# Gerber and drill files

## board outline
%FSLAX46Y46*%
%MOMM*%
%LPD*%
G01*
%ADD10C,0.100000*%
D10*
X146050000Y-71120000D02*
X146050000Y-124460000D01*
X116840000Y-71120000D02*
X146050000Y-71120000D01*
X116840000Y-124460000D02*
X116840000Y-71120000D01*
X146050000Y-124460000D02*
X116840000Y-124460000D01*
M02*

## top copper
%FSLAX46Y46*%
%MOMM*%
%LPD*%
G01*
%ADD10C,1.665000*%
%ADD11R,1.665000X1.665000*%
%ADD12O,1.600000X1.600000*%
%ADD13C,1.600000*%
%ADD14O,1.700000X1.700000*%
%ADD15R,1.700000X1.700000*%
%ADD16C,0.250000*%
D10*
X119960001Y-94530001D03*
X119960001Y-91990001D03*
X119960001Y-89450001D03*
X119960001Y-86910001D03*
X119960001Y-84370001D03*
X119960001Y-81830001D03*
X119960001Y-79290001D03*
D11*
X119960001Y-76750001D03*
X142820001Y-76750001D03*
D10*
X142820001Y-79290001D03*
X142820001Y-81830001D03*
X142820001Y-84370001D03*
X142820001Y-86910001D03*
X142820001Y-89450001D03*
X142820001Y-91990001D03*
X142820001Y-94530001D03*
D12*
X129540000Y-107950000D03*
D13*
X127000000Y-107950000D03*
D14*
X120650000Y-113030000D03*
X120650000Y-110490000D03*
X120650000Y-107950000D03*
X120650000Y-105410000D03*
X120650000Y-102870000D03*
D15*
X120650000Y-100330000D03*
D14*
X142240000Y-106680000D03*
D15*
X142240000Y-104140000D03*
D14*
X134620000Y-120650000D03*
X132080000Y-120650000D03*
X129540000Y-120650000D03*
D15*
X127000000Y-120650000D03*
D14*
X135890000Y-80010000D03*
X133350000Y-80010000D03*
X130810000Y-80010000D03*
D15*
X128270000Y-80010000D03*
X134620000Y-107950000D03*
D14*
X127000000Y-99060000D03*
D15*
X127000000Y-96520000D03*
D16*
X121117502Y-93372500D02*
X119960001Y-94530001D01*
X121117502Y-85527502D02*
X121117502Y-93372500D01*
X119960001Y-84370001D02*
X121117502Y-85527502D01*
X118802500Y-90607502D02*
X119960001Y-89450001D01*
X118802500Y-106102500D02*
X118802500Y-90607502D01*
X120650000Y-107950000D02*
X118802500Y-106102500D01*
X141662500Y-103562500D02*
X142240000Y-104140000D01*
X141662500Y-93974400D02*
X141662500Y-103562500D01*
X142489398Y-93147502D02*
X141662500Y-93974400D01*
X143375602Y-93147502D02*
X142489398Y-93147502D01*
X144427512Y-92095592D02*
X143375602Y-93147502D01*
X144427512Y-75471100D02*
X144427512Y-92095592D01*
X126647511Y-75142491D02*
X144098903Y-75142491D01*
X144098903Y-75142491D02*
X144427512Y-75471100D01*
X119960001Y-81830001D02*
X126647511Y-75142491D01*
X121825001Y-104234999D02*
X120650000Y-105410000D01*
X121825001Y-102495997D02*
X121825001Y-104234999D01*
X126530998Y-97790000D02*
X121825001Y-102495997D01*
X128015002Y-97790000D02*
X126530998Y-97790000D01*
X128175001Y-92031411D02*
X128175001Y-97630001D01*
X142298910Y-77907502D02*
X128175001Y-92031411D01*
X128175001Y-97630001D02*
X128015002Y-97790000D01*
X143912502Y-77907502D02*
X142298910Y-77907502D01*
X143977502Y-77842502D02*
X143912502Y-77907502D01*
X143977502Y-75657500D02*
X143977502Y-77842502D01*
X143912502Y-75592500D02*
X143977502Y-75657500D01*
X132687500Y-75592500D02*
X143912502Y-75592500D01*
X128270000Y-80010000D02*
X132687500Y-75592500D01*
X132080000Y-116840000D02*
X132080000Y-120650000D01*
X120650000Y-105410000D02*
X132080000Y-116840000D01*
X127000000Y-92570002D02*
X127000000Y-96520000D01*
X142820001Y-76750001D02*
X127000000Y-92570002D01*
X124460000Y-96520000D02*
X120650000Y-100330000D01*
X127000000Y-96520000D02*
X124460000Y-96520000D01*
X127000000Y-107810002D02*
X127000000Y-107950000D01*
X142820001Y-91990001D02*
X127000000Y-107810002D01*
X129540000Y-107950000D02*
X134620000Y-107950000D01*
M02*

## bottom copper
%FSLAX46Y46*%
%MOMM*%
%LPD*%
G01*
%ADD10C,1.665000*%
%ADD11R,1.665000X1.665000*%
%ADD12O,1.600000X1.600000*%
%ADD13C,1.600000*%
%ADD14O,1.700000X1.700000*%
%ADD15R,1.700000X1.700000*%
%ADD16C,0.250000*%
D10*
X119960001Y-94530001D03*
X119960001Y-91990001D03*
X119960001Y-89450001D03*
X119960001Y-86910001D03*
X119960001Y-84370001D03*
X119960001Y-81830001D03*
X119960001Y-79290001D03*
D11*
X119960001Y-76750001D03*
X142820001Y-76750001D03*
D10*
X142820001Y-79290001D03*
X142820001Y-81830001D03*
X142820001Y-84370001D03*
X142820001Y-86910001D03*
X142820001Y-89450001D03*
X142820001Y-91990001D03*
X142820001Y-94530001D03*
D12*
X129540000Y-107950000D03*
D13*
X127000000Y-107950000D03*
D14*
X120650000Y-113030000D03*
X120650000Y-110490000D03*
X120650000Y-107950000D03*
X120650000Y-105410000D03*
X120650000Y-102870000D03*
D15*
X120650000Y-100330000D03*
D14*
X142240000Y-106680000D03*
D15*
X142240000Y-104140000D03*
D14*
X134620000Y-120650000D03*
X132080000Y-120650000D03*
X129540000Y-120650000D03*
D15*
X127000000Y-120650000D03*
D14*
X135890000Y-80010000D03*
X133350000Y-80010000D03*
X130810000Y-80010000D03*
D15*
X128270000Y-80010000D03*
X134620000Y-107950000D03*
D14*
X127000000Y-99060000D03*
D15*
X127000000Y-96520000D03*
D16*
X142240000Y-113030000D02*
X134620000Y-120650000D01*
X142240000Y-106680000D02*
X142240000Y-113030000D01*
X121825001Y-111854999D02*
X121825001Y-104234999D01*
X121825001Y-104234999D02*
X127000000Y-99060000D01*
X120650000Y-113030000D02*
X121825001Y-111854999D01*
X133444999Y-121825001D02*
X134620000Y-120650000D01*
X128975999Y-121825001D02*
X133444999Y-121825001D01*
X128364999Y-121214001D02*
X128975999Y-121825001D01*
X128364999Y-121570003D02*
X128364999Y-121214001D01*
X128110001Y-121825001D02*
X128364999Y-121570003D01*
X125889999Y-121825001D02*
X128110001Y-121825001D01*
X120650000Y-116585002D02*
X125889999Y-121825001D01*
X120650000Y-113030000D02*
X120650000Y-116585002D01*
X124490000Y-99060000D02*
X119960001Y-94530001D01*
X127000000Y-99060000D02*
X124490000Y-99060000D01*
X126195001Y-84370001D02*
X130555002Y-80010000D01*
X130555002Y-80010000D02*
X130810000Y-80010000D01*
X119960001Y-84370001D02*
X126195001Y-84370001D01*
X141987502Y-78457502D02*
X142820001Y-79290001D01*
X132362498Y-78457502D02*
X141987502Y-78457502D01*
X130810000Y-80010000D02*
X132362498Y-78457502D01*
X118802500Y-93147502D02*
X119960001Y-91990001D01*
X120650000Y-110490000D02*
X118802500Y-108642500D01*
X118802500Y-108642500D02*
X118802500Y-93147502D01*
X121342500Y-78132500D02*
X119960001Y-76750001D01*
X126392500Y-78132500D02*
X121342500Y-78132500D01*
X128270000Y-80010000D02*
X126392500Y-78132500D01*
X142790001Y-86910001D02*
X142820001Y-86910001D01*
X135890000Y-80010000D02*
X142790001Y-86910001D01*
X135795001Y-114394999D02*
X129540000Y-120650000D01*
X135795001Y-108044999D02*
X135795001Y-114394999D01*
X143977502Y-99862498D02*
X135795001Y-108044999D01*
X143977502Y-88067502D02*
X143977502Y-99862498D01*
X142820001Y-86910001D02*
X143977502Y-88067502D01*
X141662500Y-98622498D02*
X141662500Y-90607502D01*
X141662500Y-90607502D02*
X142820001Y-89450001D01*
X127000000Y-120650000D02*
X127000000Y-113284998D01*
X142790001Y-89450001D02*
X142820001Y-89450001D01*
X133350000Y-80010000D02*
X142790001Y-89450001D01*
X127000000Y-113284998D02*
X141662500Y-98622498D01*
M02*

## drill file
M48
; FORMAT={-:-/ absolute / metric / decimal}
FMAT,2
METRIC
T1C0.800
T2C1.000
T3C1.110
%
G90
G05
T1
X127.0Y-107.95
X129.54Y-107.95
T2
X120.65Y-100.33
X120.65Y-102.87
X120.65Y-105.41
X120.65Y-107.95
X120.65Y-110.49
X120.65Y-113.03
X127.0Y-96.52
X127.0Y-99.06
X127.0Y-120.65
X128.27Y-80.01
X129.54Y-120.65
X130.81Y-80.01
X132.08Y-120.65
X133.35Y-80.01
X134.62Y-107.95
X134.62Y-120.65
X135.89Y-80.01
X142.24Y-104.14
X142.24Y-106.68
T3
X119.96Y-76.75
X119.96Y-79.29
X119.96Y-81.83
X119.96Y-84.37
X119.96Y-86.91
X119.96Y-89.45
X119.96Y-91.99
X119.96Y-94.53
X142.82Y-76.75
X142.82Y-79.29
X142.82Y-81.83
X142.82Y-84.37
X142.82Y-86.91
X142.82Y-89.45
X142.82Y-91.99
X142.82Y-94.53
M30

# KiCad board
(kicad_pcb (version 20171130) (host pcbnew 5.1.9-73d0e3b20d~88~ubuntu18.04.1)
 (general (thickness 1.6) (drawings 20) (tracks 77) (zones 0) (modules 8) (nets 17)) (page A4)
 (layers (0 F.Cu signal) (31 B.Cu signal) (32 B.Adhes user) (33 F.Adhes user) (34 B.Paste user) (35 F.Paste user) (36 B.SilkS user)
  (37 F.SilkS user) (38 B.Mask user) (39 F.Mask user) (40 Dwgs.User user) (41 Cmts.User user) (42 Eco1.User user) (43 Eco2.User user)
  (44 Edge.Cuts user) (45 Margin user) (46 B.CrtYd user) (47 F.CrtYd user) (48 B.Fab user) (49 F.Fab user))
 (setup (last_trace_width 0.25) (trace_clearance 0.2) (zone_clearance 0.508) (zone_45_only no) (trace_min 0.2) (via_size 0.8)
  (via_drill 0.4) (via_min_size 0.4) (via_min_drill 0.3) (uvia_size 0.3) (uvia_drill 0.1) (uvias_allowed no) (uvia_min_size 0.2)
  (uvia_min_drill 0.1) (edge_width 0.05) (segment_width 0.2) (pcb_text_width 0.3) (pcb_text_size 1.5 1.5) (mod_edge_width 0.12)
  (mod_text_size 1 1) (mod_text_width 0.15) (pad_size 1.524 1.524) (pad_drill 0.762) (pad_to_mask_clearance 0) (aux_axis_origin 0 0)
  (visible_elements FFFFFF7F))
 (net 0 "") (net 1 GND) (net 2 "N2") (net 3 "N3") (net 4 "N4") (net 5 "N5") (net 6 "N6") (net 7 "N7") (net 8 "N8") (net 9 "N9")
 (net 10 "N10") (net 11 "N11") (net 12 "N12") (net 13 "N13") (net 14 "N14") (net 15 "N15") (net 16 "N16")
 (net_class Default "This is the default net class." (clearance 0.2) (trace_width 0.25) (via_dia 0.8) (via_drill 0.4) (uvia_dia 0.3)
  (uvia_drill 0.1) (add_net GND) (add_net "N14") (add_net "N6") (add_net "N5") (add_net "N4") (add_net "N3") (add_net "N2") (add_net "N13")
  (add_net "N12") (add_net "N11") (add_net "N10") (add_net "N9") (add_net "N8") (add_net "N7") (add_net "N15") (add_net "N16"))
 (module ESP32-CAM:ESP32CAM (layer B.Cu) (at 142.820001 94.530001 180)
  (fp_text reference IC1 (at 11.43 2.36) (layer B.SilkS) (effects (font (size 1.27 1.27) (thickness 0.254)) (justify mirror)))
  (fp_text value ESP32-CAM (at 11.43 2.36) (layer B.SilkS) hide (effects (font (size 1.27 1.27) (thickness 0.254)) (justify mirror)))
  (pad 16 thru_hole circle (at 22.86 0 90) (size 1.665 1.665) (drill 1.11) (layers *.Cu *.Mask B.SilkS) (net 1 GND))
  (pad 15 thru_hole circle (at 22.86 2.54 90) (size 1.665 1.665) (drill 1.11) (layers *.Cu *.Mask B.SilkS) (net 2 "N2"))
  (pad 14 thru_hole circle (at 22.86 5.08 90) (size 1.665 1.665) (drill 1.11) (layers *.Cu *.Mask B.SilkS) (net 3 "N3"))
  (pad 13 thru_hole circle (at 22.86 7.62 90) (size 1.665 1.665) (drill 1.11) (layers *.Cu *.Mask B.SilkS) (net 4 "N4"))
  (pad 12 thru_hole circle (at 22.86 10.16 90) (size 1.665 1.665) (drill 1.11) (layers *.Cu *.Mask B.SilkS) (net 1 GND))
  (pad 11 thru_hole circle (at 22.86 12.7 90) (size 1.665 1.665) (drill 1.11) (layers *.Cu *.Mask B.SilkS) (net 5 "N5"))
  (pad 10 thru_hole circle (at 22.86 15.24 90) (size 1.665 1.665) (drill 1.11) (layers *.Cu *.Mask B.SilkS) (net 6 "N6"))
  (pad 9 thru_hole rect (at 22.86 17.78 90) (size 1.665 1.665) (drill 1.11) (layers *.Cu *.Mask B.SilkS) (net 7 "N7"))
  (pad 8 thru_hole rect (at 0 17.78 90) (size 1.665 1.665) (drill 1.11) (layers *.Cu *.Mask B.SilkS) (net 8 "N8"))
  (pad 7 thru_hole circle (at 0 15.24 90) (size 1.665 1.665) (drill 1.11) (layers *.Cu *.Mask B.SilkS) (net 1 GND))
  (pad 6 thru_hole circle (at 0 12.7 90) (size 1.665 1.665) (drill 1.11) (layers *.Cu *.Mask B.SilkS) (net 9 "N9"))
  (pad 5 thru_hole circle (at 0 10.16 90) (size 1.665 1.665) (drill 1.11) (layers *.Cu *.Mask B.SilkS) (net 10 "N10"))
  (pad 4 thru_hole circle (at 0 7.62 90) (size 1.665 1.665) (drill 1.11) (layers *.Cu *.Mask B.SilkS) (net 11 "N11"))
  (pad 3 thru_hole circle (at 0 5.08 90) (size 1.665 1.665) (drill 1.11) (layers *.Cu *.Mask B.SilkS) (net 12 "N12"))
  (pad 2 thru_hole circle (at 0 2.54 90) (size 1.665 1.665) (drill 1.11) (layers *.Cu *.Mask B.SilkS) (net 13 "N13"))
  (pad 1 thru_hole circle (at 0 0 90) (size 1.665 1.665) (drill 1.11) (layers *.Cu *.Mask B.SilkS) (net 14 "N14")))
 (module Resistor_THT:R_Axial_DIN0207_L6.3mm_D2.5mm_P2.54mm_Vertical (layer F.Cu) (at 127 107.95)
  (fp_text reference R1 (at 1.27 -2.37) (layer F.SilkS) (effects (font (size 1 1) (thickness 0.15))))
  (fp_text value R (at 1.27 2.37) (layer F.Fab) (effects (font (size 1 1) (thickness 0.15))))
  (pad 2 thru_hole oval (at 2.54 0) (size 1.6 1.6) (drill 0.8) (layers *.Cu *.Mask) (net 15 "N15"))
  (pad 1 thru_hole circle (at 0 0) (size 1.6 1.6) (drill 0.8) (layers *.Cu *.Mask) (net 13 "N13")))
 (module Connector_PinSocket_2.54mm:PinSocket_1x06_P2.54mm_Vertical (layer F.Cu) (at 120.65 100.33)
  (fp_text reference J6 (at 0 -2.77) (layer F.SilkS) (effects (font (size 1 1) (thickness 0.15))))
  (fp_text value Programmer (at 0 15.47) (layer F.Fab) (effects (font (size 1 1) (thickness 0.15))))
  (pad 6 thru_hole oval (at 0 12.7) (size 1.7 1.7) (drill 1) (layers *.Cu *.Mask) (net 1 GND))
  (pad 5 thru_hole oval (at 0 10.16) (size 1.7 1.7) (drill 1) (layers *.Cu *.Mask) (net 2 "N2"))
  (pad 4 thru_hole oval (at 0 7.62) (size 1.7 1.7) (drill 1) (layers *.Cu *.Mask) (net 3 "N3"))
  (pad 3 thru_hole oval (at 0 5.08) (size 1.7 1.7) (drill 1) (layers *.Cu *.Mask) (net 7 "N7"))
  (pad 2 thru_hole oval (at 0 2.54) (size 1.7 1.7) (drill 1) (layers *.Cu *.Mask) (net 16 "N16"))
  (pad 1 thru_hole rect (at 0 0) (size 1.7 1.7) (drill 1) (layers *.Cu *.Mask) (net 8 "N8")))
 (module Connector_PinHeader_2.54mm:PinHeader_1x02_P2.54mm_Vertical (layer F.Cu) (at 142.24 104.14)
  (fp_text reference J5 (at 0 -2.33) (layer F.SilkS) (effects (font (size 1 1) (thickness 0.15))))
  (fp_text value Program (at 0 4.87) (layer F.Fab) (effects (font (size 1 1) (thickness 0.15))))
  (pad 2 thru_hole oval (at 0 2.54) (size 1.7 1.7) (drill 1) (layers *.Cu *.Mask) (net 1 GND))
  (pad 1 thru_hole rect (at 0 0) (size 1.7 1.7) (drill 1) (layers *.Cu *.Mask) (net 5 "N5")))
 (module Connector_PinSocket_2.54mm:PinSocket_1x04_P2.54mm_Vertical (layer F.Cu) (at 127 120.65 90)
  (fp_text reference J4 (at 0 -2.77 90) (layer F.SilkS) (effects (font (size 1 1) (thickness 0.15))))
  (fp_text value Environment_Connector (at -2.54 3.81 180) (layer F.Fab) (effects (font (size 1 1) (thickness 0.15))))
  (pad 4 thru_hole oval (at 0 7.62 90) (size 1.7 1.7) (drill 1) (layers *.Cu *.Mask) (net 1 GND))
  (pad 3 thru_hole oval (at 0 5.08 90) (size 1.7 1.7) (drill 1) (layers *.Cu *.Mask) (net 7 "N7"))
  (pad 2 thru_hole oval (at 0 2.54 90) (size 1.7 1.7) (drill 1) (layers *.Cu *.Mask) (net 11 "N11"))
  (pad 1 thru_hole rect (at 0 0 90) (size 1.7 1.7) (drill 1) (layers *.Cu *.Mask) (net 12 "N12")))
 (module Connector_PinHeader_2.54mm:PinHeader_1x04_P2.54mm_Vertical (layer F.Cu) (at 128.27 80.01 90)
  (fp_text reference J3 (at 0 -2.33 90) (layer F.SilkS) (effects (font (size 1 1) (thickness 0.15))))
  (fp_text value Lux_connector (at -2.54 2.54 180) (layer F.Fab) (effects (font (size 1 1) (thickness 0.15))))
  (pad 4 thru_hole oval (at 0 7.62 90) (size 1.7 1.7) (drill 1) (layers *.Cu *.Mask) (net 11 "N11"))
  (pad 3 thru_hole oval (at 0 5.08 90) (size 1.7 1.7) (drill 1) (layers *.Cu *.Mask) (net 12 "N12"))
  (pad 2 thru_hole oval (at 0 2.54 90) (size 1.7 1.7) (drill 1) (layers *.Cu *.Mask) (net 1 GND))
  (pad 1 thru_hole rect (at 0 0 90) (size 1.7 1.7) (drill 1) (layers *.Cu *.Mask) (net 7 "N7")))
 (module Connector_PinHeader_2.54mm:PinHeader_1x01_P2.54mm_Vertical (layer F.Cu) (at 134.62 107.95)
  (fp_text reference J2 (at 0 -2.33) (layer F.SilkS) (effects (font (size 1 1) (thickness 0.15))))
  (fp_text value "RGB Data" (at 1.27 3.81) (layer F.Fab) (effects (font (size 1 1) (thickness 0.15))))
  (pad 1 thru_hole rect (at 0 0) (size 1.7 1.7) (drill 1) (layers *.Cu *.Mask) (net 15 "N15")))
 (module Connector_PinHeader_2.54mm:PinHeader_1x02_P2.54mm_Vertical (layer F.Cu) (at 127 96.52)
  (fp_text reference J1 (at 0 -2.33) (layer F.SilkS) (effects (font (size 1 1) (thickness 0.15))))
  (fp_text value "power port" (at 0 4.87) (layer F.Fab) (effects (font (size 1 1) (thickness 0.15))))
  (pad 2 thru_hole oval (at 0 2.54) (size 1.7 1.7) (drill 1) (layers *.Cu *.Mask) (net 1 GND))
  (pad 1 thru_hole rect (at 0 0) (size 1.7 1.7) (drill 1) (layers *.Cu *.Mask) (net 8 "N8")))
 (gr_line (start 146.05 71.12) (end 146.05 124.46) (layer Edge.Cuts) (width 0.1))
 (gr_line (start 116.84 71.12) (end 146.05 71.12) (layer Edge.Cuts) (width 0.1))
 (gr_line (start 116.84 124.46) (end 116.84 71.12) (layer Edge.Cuts) (width 0.1))
 (gr_line (start 146.05 124.46) (end 116.84 124.46) (layer Edge.Cuts) (width 0.1))
 (segment (start 142.24 113.03) (end 134.62 120.65) (width 0.25) (layer B.Cu) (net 1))
 (segment (start 142.24 106.68) (end 142.24 113.03) (width 0.25) (layer B.Cu) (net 1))
 (segment (start 121.825001 111.854999) (end 121.825001 104.234999) (width 0.25) (layer B.Cu) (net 1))
 (segment (start 121.825001 104.234999) (end 127 99.06) (width 0.25) (layer B.Cu) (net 1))
 (segment (start 120.65 113.03) (end 121.825001 111.854999) (width 0.25) (layer B.Cu) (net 1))
 (segment (start 133.444999 121.825001) (end 134.62 120.65) (width 0.25) (layer B.Cu) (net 1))
 (segment (start 128.975999 121.825001) (end 133.444999 121.825001) (width 0.25) (layer B.Cu) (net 1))
 (segment (start 128.364999 121.214001) (end 128.975999 121.825001) (width 0.25) (layer B.Cu) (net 1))
 (segment (start 128.364999 121.570003) (end 128.364999 121.214001) (width 0.25) (layer B.Cu) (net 1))
 (segment (start 128.110001 121.825001) (end 128.364999 121.570003) (width 0.25) (layer B.Cu) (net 1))
 (segment (start 125.889999 121.825001) (end 128.110001 121.825001) (width 0.25) (layer B.Cu) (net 1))
 (segment (start 120.65 116.585002) (end 125.889999 121.825001) (width 0.25) (layer B.Cu) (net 1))
 (segment (start 120.65 113.03) (end 120.65 116.585002) (width 0.25) (layer B.Cu) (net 1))
 (segment (start 124.49 99.06) (end 119.960001 94.530001) (width 0.25) (layer B.Cu) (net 1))
 (segment (start 127 99.06) (end 124.49 99.06) (width 0.25) (layer B.Cu) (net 1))
 (segment (start 126.195001 84.370001) (end 130.555002 80.01) (width 0.25) (layer B.Cu) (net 1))
 (segment (start 130.555002 80.01) (end 130.81 80.01) (width 0.25) (layer B.Cu) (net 1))
 (segment (start 119.960001 84.370001) (end 126.195001 84.370001) (width 0.25) (layer B.Cu) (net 1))
 (segment (start 141.987502 78.457502) (end 142.820001 79.290001) (width 0.25) (layer B.Cu) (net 1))
 (segment (start 132.362498 78.457502) (end 141.987502 78.457502) (width 0.25) (layer B.Cu) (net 1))
 (segment (start 130.81 80.01) (end 132.362498 78.457502) (width 0.25) (layer B.Cu) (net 1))
 (segment (start 121.117502 93.3725) (end 119.960001 94.530001) (width 0.25) (layer F.Cu) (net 1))
 (segment (start 121.117502 85.527502) (end 121.117502 93.3725) (width 0.25) (layer F.Cu) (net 1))
 (segment (start 119.960001 84.370001) (end 121.117502 85.527502) (width 0.25) (layer F.Cu) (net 1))
 (segment (start 118.8025 93.147502) (end 119.960001 91.990001) (width 0.25) (layer B.Cu) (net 2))
 (segment (start 120.65 110.49) (end 118.8025 108.6425) (width 0.25) (layer B.Cu) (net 2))
 (segment (start 118.8025 108.6425) (end 118.8025 93.147502) (width 0.25) (layer B.Cu) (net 2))
 (segment (start 118.8025 90.607502) (end 119.960001 89.450001) (width 0.25) (layer F.Cu) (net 3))
 (segment (start 118.8025 106.1025) (end 118.8025 90.607502) (width 0.25) (layer F.Cu) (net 3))
 (segment (start 120.65 107.95) (end 118.8025 106.1025) (width 0.25) (layer F.Cu) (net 3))
 (segment (start 141.6625 103.5625) (end 142.24 104.14) (width 0.25) (layer F.Cu) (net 5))
 (segment (start 141.6625 93.9744) (end 141.6625 103.5625) (width 0.25) (layer F.Cu) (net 5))
 (segment (start 142.489398 93.147502) (end 141.6625 93.9744) (width 0.25) (layer F.Cu) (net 5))
 (segment (start 143.375602 93.147502) (end 142.489398 93.147502) (width 0.25) (layer F.Cu) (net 5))
 (segment (start 144.427512 92.095592) (end 143.375602 93.147502) (width 0.25) (layer F.Cu) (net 5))
 (segment (start 144.427512 75.4711) (end 144.427512 92.095592) (width 0.25) (layer F.Cu) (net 5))
 (segment (start 126.647511 75.142491) (end 144.098903 75.142491) (width 0.25) (layer F.Cu) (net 5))
 (segment (start 144.098903 75.142491) (end 144.427512 75.4711) (width 0.25) (layer F.Cu) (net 5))
 (segment (start 119.960001 81.830001) (end 126.647511 75.142491) (width 0.25) (layer F.Cu) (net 5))
 (segment (start 121.3425 78.1325) (end 119.960001 76.750001) (width 0.25) (layer B.Cu) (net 7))
 (segment (start 126.3925 78.1325) (end 121.3425 78.1325) (width 0.25) (layer B.Cu) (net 7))
 (segment (start 128.27 80.01) (end 126.3925 78.1325) (width 0.25) (layer B.Cu) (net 7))
 (segment (start 121.825001 104.234999) (end 120.65 105.41) (width 0.25) (layer F.Cu) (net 7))
 (segment (start 121.825001 102.495997) (end 121.825001 104.234999) (width 0.25) (layer F.Cu) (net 7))
 (segment (start 126.530998 97.79) (end 121.825001 102.495997) (width 0.25) (layer F.Cu) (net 7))
 (segment (start 128.015002 97.79) (end 126.530998 97.79) (width 0.25) (layer F.Cu) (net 7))
 (segment (start 128.175001 92.031411) (end 128.175001 97.630001) (width 0.25) (layer F.Cu) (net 7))
 (segment (start 142.29891 77.907502) (end 128.175001 92.031411) (width 0.25) (layer F.Cu) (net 7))
 (segment (start 128.175001 97.630001) (end 128.015002 97.79) (width 0.25) (layer F.Cu) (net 7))
 (segment (start 143.912502 77.907502) (end 142.29891 77.907502) (width 0.25) (layer F.Cu) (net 7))
 (segment (start 143.977502 77.842502) (end 143.912502 77.907502) (width 0.25) (layer F.Cu) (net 7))
 (segment (start 143.977502 75.6575) (end 143.977502 77.842502) (width 0.25) (layer F.Cu) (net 7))
 (segment (start 143.912502 75.5925) (end 143.977502 75.6575) (width 0.25) (layer F.Cu) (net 7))
 (segment (start 132.6875 75.5925) (end 143.912502 75.5925) (width 0.25) (layer F.Cu) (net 7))
 (segment (start 128.27 80.01) (end 132.6875 75.5925) (width 0.25) (layer F.Cu) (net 7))
 (segment (start 132.08 116.84) (end 132.08 120.65) (width 0.25) (layer F.Cu) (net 7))
 (segment (start 120.65 105.41) (end 132.08 116.84) (width 0.25) (layer F.Cu) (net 7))
 (segment (start 127 92.570002) (end 127 96.52) (width 0.25) (layer F.Cu) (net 8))
 (segment (start 142.820001 76.750001) (end 127 92.570002) (width 0.25) (layer F.Cu) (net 8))
 (segment (start 124.46 96.52) (end 120.65 100.33) (width 0.25) (layer F.Cu) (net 8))
 (segment (start 127 96.52) (end 124.46 96.52) (width 0.25) (layer F.Cu) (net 8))
 (segment (start 142.790001 86.910001) (end 142.820001 86.910001) (width 0.25) (layer B.Cu) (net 11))
 (segment (start 135.89 80.01) (end 142.790001 86.910001) (width 0.25) (layer B.Cu) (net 11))
 (segment (start 135.795001 114.394999) (end 129.54 120.65) (width 0.25) (layer B.Cu) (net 11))
 (segment (start 135.795001 108.044999) (end 135.795001 114.394999) (width 0.25) (layer B.Cu) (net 11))
 (segment (start 143.977502 99.862498) (end 135.795001 108.044999) (width 0.25) (layer B.Cu) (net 11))
 (segment (start 143.977502 88.067502) (end 143.977502 99.862498) (width 0.25) (layer B.Cu) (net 11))
 (segment (start 142.820001 86.910001) (end 143.977502 88.067502) (width 0.25) (layer B.Cu) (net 11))
 (segment (start 141.6625 98.622498) (end 141.6625 90.607502) (width 0.25) (layer B.Cu) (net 12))
 (segment (start 141.6625 90.607502) (end 142.820001 89.450001) (width 0.25) (layer B.Cu) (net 12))
 (segment (start 127 120.65) (end 127 113.284998) (width 0.25) (layer B.Cu) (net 12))
 (segment (start 142.790001 89.450001) (end 142.820001 89.450001) (width 0.25) (layer B.Cu) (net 12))
 (segment (start 133.35 80.01) (end 142.790001 89.450001) (width 0.25) (layer B.Cu) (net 12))
 (segment (start 127 113.284998) (end 141.6625 98.622498) (width 0.25) (layer B.Cu) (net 12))
 (segment (start 127 107.810002) (end 127 107.95) (width 0.25) (layer F.Cu) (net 13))
 (segment (start 142.820001 91.990001) (end 127 107.810002) (width 0.25) (layer F.Cu) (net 13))
 (segment (start 129.54 107.95) (end 134.62 107.95) (width 0.25) (layer F.Cu) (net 15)))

